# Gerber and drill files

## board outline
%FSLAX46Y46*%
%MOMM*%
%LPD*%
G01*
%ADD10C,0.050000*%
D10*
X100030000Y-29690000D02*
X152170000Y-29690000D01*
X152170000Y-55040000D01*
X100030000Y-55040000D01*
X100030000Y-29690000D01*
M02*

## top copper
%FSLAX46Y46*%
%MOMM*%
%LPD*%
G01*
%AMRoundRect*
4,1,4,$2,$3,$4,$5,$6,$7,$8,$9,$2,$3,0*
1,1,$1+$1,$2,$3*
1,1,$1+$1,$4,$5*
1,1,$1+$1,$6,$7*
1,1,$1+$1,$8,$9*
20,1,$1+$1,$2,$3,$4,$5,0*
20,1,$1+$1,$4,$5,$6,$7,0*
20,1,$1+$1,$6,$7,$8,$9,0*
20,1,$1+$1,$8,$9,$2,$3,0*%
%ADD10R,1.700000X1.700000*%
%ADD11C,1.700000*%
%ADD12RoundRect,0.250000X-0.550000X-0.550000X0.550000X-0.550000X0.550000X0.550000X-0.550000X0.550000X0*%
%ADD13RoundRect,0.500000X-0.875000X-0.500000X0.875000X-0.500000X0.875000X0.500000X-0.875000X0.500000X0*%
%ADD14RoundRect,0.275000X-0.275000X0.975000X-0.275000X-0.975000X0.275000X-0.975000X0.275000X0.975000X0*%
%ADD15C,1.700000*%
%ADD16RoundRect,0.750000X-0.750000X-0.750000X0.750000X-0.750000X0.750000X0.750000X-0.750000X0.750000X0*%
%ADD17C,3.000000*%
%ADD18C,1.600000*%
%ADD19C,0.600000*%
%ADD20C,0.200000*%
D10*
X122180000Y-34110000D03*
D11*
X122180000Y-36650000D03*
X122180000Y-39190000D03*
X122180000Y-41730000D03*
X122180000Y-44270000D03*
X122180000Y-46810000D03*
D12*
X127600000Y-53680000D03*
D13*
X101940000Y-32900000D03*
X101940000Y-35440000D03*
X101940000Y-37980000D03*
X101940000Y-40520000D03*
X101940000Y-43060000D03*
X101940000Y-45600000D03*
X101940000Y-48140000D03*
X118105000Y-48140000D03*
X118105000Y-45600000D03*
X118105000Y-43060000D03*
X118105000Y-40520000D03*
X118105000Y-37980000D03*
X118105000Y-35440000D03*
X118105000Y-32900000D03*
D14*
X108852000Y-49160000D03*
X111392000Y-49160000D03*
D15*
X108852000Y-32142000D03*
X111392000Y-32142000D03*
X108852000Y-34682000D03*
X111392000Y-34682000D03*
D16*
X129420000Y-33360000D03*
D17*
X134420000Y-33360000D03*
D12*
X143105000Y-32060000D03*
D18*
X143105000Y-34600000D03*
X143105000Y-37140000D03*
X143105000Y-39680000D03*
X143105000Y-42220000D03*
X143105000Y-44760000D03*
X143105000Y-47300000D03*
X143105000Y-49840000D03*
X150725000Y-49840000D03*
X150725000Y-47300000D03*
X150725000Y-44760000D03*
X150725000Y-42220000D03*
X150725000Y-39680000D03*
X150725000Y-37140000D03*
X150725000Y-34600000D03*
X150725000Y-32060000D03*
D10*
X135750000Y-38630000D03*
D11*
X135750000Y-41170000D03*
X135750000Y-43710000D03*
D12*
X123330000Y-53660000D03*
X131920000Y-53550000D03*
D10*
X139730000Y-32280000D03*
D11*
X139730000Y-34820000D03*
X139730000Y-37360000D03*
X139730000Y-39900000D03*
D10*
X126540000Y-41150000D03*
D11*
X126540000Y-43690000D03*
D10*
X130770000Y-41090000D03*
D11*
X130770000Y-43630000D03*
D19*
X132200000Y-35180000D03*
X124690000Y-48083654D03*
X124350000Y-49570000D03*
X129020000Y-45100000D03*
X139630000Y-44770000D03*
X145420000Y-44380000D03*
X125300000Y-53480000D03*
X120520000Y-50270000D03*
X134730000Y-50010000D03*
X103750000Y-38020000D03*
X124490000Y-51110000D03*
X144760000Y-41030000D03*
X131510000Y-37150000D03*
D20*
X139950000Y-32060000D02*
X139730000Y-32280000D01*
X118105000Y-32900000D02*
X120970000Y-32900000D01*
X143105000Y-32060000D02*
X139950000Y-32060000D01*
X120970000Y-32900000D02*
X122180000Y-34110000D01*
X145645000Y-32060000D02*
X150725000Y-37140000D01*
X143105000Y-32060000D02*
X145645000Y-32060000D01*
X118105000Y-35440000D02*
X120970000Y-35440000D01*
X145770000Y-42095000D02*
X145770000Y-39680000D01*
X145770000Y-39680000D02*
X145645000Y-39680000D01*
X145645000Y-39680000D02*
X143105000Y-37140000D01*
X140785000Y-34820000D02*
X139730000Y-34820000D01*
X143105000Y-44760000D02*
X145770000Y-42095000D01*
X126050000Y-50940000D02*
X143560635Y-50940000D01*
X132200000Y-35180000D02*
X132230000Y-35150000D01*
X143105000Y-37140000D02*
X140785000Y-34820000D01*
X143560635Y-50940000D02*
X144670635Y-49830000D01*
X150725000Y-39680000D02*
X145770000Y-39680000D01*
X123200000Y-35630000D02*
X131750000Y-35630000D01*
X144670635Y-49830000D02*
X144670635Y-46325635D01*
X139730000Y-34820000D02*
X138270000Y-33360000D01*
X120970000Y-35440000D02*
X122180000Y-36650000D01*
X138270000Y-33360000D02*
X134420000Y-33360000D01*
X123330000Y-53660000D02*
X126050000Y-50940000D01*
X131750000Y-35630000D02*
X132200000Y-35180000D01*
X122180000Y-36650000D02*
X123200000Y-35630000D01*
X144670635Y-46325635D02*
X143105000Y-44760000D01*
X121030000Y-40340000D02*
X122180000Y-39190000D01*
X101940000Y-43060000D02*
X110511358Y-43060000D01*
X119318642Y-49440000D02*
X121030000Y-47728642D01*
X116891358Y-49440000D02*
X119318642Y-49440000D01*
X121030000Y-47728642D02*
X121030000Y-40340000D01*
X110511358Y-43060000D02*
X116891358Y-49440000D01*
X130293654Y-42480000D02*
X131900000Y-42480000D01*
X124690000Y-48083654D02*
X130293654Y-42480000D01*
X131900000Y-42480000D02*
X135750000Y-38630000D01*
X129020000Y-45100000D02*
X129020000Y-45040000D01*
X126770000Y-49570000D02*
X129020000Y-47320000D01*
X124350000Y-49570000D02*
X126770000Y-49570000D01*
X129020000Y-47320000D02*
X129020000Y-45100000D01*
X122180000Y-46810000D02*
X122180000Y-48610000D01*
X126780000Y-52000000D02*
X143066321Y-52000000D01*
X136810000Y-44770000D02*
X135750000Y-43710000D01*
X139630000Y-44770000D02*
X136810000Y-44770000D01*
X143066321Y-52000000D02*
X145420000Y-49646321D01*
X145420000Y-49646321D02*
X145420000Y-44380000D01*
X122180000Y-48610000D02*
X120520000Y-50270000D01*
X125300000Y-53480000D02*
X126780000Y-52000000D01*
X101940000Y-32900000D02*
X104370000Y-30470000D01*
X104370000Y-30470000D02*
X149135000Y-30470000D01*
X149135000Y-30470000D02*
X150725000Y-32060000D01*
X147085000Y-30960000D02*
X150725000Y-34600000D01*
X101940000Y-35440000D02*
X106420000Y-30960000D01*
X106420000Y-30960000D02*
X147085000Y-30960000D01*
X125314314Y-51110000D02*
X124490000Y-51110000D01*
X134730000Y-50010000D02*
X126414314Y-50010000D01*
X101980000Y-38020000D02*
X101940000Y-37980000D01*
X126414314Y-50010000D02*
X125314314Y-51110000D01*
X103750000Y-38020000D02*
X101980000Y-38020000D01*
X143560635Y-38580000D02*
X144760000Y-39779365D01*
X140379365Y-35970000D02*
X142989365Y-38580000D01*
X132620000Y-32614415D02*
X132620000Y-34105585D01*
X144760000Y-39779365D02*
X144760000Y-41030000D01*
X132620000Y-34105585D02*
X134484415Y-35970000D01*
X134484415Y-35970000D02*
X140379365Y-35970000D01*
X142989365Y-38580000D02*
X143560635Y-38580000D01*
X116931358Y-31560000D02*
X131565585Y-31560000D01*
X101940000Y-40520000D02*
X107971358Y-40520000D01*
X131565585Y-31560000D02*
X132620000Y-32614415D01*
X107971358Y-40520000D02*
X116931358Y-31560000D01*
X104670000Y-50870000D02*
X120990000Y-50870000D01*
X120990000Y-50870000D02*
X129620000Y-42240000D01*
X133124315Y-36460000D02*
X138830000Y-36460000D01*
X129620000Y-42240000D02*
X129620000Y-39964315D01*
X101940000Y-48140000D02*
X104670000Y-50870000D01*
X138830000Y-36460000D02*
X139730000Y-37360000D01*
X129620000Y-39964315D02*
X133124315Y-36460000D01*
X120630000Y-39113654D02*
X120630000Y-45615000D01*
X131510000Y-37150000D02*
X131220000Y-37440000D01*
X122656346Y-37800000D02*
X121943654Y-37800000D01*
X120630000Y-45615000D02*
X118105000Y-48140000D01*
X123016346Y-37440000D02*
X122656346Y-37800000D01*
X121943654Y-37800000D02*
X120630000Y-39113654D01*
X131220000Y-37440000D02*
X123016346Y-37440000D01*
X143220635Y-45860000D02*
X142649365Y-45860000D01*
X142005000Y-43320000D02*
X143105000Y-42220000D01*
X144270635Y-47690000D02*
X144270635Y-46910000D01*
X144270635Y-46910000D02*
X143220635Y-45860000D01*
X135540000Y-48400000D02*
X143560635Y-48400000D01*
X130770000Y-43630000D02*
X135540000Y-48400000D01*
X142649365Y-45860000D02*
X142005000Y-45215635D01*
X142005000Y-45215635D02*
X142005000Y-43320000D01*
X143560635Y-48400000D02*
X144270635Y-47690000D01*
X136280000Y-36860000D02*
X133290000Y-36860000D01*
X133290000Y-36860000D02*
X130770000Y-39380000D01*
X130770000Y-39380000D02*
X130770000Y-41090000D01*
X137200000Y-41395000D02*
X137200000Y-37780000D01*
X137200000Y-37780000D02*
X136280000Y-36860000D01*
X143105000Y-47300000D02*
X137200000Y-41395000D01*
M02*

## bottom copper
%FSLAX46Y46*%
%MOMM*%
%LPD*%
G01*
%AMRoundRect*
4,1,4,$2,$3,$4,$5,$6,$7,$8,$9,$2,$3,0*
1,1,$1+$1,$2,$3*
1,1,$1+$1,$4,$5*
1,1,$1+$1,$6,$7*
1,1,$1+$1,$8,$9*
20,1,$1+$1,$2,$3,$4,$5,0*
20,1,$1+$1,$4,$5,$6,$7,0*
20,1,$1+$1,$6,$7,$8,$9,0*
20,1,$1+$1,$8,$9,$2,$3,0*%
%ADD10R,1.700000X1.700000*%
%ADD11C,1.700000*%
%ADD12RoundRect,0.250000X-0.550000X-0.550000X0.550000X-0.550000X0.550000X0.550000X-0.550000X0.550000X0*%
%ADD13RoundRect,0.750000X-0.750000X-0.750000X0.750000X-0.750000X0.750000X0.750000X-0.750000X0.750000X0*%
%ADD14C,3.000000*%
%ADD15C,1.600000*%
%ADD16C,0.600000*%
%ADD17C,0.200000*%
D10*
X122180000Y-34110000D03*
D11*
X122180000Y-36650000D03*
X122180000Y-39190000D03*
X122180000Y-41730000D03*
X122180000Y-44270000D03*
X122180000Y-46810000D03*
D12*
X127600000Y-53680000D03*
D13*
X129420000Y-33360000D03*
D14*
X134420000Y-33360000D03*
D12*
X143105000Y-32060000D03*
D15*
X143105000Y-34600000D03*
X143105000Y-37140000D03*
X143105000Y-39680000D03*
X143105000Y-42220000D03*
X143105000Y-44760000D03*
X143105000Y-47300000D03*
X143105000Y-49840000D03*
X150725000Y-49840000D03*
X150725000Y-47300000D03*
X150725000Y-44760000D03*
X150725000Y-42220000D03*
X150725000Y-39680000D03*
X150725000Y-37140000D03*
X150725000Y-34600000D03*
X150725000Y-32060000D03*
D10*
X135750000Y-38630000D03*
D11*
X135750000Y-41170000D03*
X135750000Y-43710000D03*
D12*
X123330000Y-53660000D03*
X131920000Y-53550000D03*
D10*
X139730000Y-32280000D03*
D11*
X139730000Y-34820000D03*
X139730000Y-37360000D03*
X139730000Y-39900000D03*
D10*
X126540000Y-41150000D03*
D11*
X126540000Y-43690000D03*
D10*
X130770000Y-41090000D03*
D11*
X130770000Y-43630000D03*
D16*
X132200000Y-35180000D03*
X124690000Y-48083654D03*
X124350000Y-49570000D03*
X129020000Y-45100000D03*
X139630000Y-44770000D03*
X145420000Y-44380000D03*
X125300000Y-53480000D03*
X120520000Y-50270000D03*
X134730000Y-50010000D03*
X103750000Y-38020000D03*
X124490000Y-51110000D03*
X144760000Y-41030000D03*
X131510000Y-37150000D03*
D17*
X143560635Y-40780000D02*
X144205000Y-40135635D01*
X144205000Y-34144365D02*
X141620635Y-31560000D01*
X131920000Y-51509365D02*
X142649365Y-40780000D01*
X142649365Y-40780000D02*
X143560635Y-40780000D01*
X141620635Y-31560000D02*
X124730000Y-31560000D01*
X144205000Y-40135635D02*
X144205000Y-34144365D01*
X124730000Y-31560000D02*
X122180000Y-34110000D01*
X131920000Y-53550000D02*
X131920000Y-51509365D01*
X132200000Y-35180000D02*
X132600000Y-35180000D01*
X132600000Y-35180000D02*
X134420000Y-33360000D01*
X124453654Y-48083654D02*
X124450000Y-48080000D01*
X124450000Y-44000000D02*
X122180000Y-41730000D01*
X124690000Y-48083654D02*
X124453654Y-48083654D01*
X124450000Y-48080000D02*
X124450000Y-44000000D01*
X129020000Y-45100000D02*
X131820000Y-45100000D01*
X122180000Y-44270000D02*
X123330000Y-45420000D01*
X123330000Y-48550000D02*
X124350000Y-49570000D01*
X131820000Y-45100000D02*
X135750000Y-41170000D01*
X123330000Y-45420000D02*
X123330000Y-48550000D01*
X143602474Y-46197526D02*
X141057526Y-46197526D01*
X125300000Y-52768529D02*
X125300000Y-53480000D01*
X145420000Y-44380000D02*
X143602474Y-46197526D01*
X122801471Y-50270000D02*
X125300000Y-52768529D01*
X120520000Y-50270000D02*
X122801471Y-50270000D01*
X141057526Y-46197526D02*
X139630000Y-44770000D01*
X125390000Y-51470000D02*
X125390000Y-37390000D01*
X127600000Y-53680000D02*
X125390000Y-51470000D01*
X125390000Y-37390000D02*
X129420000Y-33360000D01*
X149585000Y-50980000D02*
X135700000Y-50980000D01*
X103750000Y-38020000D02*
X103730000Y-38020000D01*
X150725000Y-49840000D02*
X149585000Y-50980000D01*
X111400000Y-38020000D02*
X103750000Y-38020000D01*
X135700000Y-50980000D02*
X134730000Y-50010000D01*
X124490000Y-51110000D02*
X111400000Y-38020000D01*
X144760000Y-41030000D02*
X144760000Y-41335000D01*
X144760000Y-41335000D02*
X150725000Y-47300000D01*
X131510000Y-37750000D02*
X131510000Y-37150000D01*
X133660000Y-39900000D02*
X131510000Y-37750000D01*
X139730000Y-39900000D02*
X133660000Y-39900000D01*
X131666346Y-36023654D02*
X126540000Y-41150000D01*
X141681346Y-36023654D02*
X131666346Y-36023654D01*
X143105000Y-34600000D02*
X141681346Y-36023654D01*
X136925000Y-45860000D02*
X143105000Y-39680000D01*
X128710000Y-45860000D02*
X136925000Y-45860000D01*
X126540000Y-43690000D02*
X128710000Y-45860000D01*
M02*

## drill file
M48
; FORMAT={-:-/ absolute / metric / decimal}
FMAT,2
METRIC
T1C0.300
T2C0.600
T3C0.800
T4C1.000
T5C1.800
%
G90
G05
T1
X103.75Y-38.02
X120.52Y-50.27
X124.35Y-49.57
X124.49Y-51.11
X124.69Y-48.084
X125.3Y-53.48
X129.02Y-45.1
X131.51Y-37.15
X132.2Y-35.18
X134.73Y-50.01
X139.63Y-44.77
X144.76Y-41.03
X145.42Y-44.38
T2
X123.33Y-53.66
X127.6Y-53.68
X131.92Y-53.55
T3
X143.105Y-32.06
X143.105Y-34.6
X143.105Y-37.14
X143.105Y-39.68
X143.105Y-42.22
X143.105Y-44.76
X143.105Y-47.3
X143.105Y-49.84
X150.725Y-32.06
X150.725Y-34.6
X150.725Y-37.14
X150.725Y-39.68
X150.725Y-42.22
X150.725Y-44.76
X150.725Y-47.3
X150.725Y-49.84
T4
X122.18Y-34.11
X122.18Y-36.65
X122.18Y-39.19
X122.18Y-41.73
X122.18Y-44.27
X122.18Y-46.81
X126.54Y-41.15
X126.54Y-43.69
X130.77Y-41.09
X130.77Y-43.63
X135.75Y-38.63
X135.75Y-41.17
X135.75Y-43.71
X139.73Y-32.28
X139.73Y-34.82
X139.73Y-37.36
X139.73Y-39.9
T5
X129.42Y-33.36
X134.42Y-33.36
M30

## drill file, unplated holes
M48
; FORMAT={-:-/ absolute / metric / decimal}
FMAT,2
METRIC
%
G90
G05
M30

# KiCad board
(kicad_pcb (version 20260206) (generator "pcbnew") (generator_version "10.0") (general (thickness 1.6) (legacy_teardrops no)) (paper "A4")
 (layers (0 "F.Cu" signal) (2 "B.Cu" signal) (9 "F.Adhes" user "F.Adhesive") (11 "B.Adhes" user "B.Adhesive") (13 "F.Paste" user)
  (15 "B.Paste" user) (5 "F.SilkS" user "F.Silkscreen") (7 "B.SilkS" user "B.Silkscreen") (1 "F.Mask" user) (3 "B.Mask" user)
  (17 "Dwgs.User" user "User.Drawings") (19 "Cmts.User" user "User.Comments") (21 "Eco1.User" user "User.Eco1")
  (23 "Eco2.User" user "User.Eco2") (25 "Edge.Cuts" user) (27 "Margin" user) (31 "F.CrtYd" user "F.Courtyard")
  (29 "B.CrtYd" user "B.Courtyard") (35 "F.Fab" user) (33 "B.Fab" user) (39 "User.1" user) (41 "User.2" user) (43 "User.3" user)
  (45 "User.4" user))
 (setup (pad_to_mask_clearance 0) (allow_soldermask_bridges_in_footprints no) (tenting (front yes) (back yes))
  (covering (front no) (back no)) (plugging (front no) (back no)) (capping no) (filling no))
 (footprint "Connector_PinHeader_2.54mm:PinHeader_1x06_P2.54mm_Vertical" (layer "F.Cu") (at 122.18 34.11)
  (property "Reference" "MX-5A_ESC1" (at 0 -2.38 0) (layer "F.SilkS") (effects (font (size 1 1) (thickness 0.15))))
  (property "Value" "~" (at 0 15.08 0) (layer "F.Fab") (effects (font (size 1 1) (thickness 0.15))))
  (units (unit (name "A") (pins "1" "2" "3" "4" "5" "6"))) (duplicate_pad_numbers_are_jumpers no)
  (pad "1" thru_hole rect (at 0 0) (size 1.7 1.7) (drill 1) (layers "*.Cu" "*.Mask") (remove_unused_layers no) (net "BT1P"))
  (pad "2" thru_hole circle (at 0 2.54) (size 1.7 1.7) (drill 1) (layers "*.Cu" "*.Mask") (remove_unused_layers no) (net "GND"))
  (pad "3" thru_hole circle (at 0 5.08) (size 1.7 1.7) (drill 1) (layers "*.Cu" "*.Mask") (remove_unused_layers no)
   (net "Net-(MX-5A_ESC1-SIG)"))
  (pad "4" thru_hole circle (at 0 7.62) (size 1.7 1.7) (drill 1) (layers "*.Cu" "*.Mask") (remove_unused_layers no)
   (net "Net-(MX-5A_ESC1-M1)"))
  (pad "5" thru_hole circle (at 0 10.16) (size 1.7 1.7) (drill 1) (layers "*.Cu" "*.Mask") (remove_unused_layers no)
   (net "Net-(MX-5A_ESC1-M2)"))
  (pad "6" thru_hole circle (at 0 12.7) (size 1.7 1.7) (drill 1) (layers "*.Cu" "*.Mask") (remove_unused_layers no)
   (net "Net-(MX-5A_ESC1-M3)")))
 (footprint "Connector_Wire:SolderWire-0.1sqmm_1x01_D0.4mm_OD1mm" (layer "F.Cu") (at 127.6 53.68)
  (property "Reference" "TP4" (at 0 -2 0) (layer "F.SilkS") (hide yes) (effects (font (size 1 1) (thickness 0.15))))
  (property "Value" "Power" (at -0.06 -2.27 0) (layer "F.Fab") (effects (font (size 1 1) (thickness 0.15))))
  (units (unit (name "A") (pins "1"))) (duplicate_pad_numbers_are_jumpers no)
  (pad "1" thru_hole roundrect (at 0 0) (size 1.6 1.6) (drill 0.6) (layers "*.Cu" "*.Mask") (remove_unused_layers no)
   (roundrect_rratio 0.15625) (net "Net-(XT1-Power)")))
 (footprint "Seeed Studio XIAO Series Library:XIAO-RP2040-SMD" (layer "F.Cu") (at 109.94 40.52)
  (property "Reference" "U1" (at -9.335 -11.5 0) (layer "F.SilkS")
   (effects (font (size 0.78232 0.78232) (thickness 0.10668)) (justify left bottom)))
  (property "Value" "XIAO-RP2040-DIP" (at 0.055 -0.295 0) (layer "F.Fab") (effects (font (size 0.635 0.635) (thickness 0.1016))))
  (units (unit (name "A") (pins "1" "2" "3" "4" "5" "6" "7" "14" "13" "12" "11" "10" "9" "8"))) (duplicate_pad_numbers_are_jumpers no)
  (pad "1" smd roundrect (at -8 -7.62) (size 2.75 2) (layers "F.Cu" "F.Mask" "F.Paste") (roundrect_rratio 0.25) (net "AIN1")
   (solder_mask_margin 0.0508) (thermal_bridge_angle 45))
  (pad "2" smd roundrect (at -8 -5.08) (size 2.75 2) (layers "F.Cu" "F.Mask" "F.Paste") (roundrect_rratio 0.25) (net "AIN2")
   (solder_mask_margin 0.0508) (thermal_bridge_angle 45))
  (pad "3" smd roundrect (at -8 -2.54) (size 2.75 2) (layers "F.Cu" "F.Mask" "F.Paste") (roundrect_rratio 0.25) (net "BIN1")
   (solder_mask_margin 0.0508) (thermal_bridge_angle 45))
  (pad "4" smd roundrect (at -8 0) (size 2.75 2) (layers "F.Cu" "F.Mask" "F.Paste") (roundrect_rratio 0.25) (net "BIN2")
   (solder_mask_margin 0.0508) (thermal_bridge_angle 45))
  (pad "5" smd roundrect (at -8 2.54) (size 2.75 2) (layers "F.Cu" "F.Mask" "F.Paste") (roundrect_rratio 0.25) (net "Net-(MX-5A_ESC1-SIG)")
   (solder_mask_margin 0.0508) (thermal_bridge_angle 45))
  (pad "6" smd roundrect (at -8 5.08) (size 2.75 2) (layers "F.Cu" "F.Mask" "F.Paste") (roundrect_rratio 0.25)
   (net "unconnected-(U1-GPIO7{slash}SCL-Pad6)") (solder_mask_margin 0.0508) (thermal_bridge_angle 45))
  (pad "7" smd roundrect (at -8 7.62) (size 2.75 2) (layers "F.Cu" "F.Mask" "F.Paste") (roundrect_rratio 0.25)
   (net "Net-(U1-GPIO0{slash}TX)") (solder_mask_margin 0.0508) (thermal_bridge_angle 45))
  (pad "8" smd roundrect (at 8.165 7.62) (size 2.75 2) (layers "F.Cu" "F.Mask" "F.Paste") (roundrect_rratio 0.25)
   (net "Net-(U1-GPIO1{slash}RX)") (solder_mask_margin 0.0508) (thermal_bridge_angle 45))
  (pad "9" smd roundrect (at 8.165 5.08) (size 2.75 2) (layers "F.Cu" "F.Mask" "F.Paste") (roundrect_rratio 0.25)
   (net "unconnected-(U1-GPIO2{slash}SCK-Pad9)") (solder_mask_margin 0.0508) (thermal_bridge_angle 45))
  (pad "10" smd roundrect (at 8.165 2.54) (size 2.75 2) (layers "F.Cu" "F.Mask" "F.Paste") (roundrect_rratio 0.25)
   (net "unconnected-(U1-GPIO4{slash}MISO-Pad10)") (solder_mask_margin 0.0508) (thermal_bridge_angle 45))
  (pad "11" smd roundrect (at 8.165 0) (size 2.75 2) (layers "F.Cu" "F.Mask" "F.Paste") (roundrect_rratio 0.25)
   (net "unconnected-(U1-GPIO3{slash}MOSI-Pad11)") (solder_mask_margin 0.0508) (thermal_bridge_angle 45))
  (pad "12" smd roundrect (at 8.165 -2.54) (size 2.75 2) (layers "F.Cu" "F.Mask" "F.Paste") (roundrect_rratio 0.25)
   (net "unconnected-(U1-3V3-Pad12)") (solder_mask_margin 0.0508) (thermal_bridge_angle 45))
  (pad "13" smd roundrect (at 8.165 -5.08) (size 2.75 2) (layers "F.Cu" "F.Mask" "F.Paste") (roundrect_rratio 0.25) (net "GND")
   (solder_mask_margin 0.0508) (thermal_bridge_angle 45))
  (pad "14" smd roundrect (at 8.165 -7.62) (size 2.75 2) (layers "F.Cu" "F.Mask" "F.Paste") (roundrect_rratio 0.25) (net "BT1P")
   (solder_mask_margin 0.0508) (thermal_bridge_angle 45))
  (pad "15" smd roundrect (at -1.088 8.64 270) (size 2.5 1.1) (layers "F.Cu" "F.Mask" "F.Paste") (roundrect_rratio 0.25)
   (thermal_bridge_angle 45))
  (pad "16" smd roundrect (at 1.452 8.64 270) (size 2.5 1.1) (layers "F.Cu" "F.Mask" "F.Paste") (roundrect_rratio 0.25)
   (thermal_bridge_angle 45))
  (pad "17" smd circle (at -1.088 -8.378) (size 1.7 1.7) (layers "F.Cu" "F.Mask" "F.Paste"))
  (pad "18" smd circle (at 1.452 -8.378) (size 1.7 1.7) (layers "F.Cu" "F.Mask" "F.Paste"))
  (pad "19" smd circle (at -1.088 -5.838) (size 1.7 1.7) (layers "F.Cu" "F.Mask" "F.Paste"))
  (pad "20" smd circle (at 1.452 -5.838) (size 1.7 1.7) (layers "F.Cu" "F.Mask" "F.Paste")))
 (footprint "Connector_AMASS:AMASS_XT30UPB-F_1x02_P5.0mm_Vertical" (layer "F.Cu") (at 129.42 33.36)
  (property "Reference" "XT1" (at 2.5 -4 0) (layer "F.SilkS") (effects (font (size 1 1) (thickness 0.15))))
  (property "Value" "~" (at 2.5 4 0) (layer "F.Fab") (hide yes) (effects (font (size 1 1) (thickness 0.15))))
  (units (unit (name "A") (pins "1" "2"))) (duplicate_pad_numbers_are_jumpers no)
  (pad "1" thru_hole roundrect (at 0 0) (size 3 3) (drill 1.8) (layers "*.Cu" "*.Mask") (remove_unused_layers no) (roundrect_rratio 0.25)
   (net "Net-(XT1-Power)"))
  (pad "2" thru_hole circle (at 5 0) (size 3 3) (drill 1.8) (layers "*.Cu" "*.Mask") (remove_unused_layers no) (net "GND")))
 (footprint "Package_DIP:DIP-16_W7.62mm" (layer "F.Cu") (at 143.105 32.06)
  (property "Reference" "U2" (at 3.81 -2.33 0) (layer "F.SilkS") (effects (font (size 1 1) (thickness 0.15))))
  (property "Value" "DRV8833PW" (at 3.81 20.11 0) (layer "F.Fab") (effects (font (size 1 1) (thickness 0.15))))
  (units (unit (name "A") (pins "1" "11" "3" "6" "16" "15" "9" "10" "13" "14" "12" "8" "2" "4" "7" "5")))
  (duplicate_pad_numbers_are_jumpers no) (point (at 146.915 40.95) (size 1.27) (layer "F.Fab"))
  (pad "1" thru_hole roundrect (at 0 0) (size 1.6 1.6) (drill 0.8) (layers "*.Cu" "*.Mask") (remove_unused_layers no)
   (roundrect_rratio 0.15625) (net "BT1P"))
  (pad "2" thru_hole circle (at 0 2.54) (size 1.6 1.6) (drill 0.8) (layers "*.Cu" "*.Mask") (remove_unused_layers no) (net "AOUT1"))
  (pad "3" thru_hole circle (at 0 5.08) (size 1.6 1.6) (drill 0.8) (layers "*.Cu" "*.Mask") (remove_unused_layers no) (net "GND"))
  (pad "4" thru_hole circle (at 0 7.62) (size 1.6 1.6) (drill 0.8) (layers "*.Cu" "*.Mask") (remove_unused_layers no) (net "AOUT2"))
  (pad "5" thru_hole circle (at 0 10.16) (size 1.6 1.6) (drill 0.8) (layers "*.Cu" "*.Mask") (remove_unused_layers no) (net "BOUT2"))
  (pad "6" thru_hole circle (at 0 12.7) (size 1.6 1.6) (drill 0.8) (layers "*.Cu" "*.Mask") (remove_unused_layers no) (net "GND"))
  (pad "7" thru_hole circle (at 0 15.24) (size 1.6 1.6) (drill 0.8) (layers "*.Cu" "*.Mask") (remove_unused_layers no) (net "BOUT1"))
  (pad "8" thru_hole circle (at 0 17.78) (size 1.6 1.6) (drill 0.8) (layers "*.Cu" "*.Mask") (remove_unused_layers no)
   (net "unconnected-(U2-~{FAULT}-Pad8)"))
  (pad "9" thru_hole circle (at 7.62 17.78) (size 1.6 1.6) (drill 0.8) (layers "*.Cu" "*.Mask") (remove_unused_layers no) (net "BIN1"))
  (pad "10" thru_hole circle (at 7.62 15.24) (size 1.6 1.6) (drill 0.8) (layers "*.Cu" "*.Mask") (remove_unused_layers no) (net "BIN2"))
  (pad "11" thru_hole circle (at 7.62 12.7) (size 1.6 1.6) (drill 0.8) (layers "*.Cu" "*.Mask") (remove_unused_layers no)
   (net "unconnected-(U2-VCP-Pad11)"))
  (pad "12" thru_hole circle (at 7.62 10.16) (size 1.6 1.6) (drill 0.8) (layers "*.Cu" "*.Mask") (remove_unused_layers no)
   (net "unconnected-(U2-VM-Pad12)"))
  (pad "13" thru_hole circle (at 7.62 7.62) (size 1.6 1.6) (drill 0.8) (layers "*.Cu" "*.Mask") (remove_unused_layers no) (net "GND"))
  (pad "14" thru_hole circle (at 7.62 5.08) (size 1.6 1.6) (drill 0.8) (layers "*.Cu" "*.Mask") (remove_unused_layers no) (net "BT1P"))
  (pad "15" thru_hole circle (at 7.62 2.54) (size 1.6 1.6) (drill 0.8) (layers "*.Cu" "*.Mask") (remove_unused_layers no) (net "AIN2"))
  (pad "16" thru_hole circle (at 7.62 0) (size 1.6 1.6) (drill 0.8) (layers "*.Cu" "*.Mask") (remove_unused_layers no) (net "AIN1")))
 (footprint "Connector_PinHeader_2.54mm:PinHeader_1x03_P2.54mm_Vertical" (layer "F.Cu") (at 135.75 38.63)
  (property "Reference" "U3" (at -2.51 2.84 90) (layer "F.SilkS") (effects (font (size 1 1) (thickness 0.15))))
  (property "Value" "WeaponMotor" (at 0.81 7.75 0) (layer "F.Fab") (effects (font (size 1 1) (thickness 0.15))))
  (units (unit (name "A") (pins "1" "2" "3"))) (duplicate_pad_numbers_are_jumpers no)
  (pad "1" thru_hole rect (at 0 0) (size 1.7 1.7) (drill 1) (layers "*.Cu" "*.Mask") (remove_unused_layers no) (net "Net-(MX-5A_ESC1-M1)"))
  (pad "2" thru_hole circle (at 0 2.54) (size 1.7 1.7) (drill 1) (layers "*.Cu" "*.Mask") (remove_unused_layers no)
   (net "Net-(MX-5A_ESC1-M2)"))
  (pad "3" thru_hole circle (at 0 5.08) (size 1.7 1.7) (drill 1) (layers "*.Cu" "*.Mask") (remove_unused_layers no)
   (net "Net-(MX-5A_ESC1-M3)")))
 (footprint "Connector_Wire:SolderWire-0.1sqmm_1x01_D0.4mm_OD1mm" (layer "F.Cu") (at 123.33 53.66)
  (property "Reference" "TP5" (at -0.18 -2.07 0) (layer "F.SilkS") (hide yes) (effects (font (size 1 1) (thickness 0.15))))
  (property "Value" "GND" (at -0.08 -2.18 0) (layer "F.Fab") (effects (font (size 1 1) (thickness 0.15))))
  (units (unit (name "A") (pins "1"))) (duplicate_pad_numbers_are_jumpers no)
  (pad "1" thru_hole roundrect (at 0 0) (size 1.6 1.6) (drill 0.6) (layers "*.Cu" "*.Mask") (remove_unused_layers no)
   (roundrect_rratio 0.15625) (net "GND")))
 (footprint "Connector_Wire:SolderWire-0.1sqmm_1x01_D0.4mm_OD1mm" (layer "F.Cu") (at 131.92 53.55)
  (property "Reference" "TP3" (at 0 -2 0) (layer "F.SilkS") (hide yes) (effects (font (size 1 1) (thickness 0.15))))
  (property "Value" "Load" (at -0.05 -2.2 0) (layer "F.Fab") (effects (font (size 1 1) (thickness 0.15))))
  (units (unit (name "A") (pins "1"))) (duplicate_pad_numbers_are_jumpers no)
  (pad "1" thru_hole roundrect (at 0 0) (size 1.6 1.6) (drill 0.6) (layers "*.Cu" "*.Mask") (remove_unused_layers no)
   (roundrect_rratio 0.15625) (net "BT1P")))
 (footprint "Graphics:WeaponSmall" (layer "F.Cu") (at 103.49791 55.032445 90)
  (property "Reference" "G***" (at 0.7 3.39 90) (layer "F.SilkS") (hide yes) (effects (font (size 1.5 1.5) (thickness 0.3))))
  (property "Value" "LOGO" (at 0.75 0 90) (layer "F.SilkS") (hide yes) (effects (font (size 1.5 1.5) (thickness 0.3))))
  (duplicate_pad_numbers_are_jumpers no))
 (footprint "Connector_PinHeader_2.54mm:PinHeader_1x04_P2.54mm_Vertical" (layer "F.Cu") (at 139.73 32.28)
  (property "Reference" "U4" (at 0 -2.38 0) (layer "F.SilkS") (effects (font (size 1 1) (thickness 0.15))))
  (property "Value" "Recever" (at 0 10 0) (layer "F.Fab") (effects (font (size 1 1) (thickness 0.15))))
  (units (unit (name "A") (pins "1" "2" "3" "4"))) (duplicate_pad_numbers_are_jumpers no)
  (pad "1" thru_hole rect (at 0 0) (size 1.7 1.7) (drill 1) (layers "*.Cu" "*.Mask") (remove_unused_layers no) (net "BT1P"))
  (pad "2" thru_hole circle (at 0 2.54) (size 1.7 1.7) (drill 1) (layers "*.Cu" "*.Mask") (remove_unused_layers no) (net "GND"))
  (pad "3" thru_hole circle (at 0 5.08) (size 1.7 1.7) (drill 1) (layers "*.Cu" "*.Mask") (remove_unused_layers no)
   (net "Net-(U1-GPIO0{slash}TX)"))
  (pad "4" thru_hole circle (at 0 7.62) (size 1.7 1.7) (drill 1) (layers "*.Cu" "*.Mask") (remove_unused_layers no)
   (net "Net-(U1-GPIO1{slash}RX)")))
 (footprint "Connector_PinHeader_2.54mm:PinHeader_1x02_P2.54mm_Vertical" (layer "F.Cu") (at 126.54 41.15)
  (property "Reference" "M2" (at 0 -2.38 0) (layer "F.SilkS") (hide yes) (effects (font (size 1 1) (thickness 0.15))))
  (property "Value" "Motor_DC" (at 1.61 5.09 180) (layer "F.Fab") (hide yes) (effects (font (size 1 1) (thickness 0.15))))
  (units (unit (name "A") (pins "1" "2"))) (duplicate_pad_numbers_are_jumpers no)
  (pad "1" thru_hole rect (at 0 0) (size 1.7 1.7) (drill 1) (layers "*.Cu" "*.Mask") (remove_unused_layers no) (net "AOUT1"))
  (pad "2" thru_hole circle (at 0 2.54) (size 1.7 1.7) (drill 1) (layers "*.Cu" "*.Mask") (remove_unused_layers no) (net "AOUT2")))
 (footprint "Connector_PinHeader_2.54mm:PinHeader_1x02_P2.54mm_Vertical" (layer "F.Cu") (at 130.77 41.09)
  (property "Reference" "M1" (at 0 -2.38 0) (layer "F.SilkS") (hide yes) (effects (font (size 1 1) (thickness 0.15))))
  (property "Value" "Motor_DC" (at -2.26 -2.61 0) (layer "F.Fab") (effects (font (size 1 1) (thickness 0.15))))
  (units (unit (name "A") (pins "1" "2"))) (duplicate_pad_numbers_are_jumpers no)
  (pad "1" thru_hole rect (at 0 0) (size 1.7 1.7) (drill 1) (layers "*.Cu" "*.Mask") (remove_unused_layers no) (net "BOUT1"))
  (pad "2" thru_hole circle (at 0 2.54) (size 1.7 1.7) (drill 1) (layers "*.Cu" "*.Mask") (remove_unused_layers no) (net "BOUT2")))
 (gr_rect (start 100.03 29.69) (end 152.17 55.04) (stroke (width 0.05) (type default)) (fill no) (layer "Edge.Cuts"))
 (segment (start 139.95 32.06) (end 139.73 32.28) (width 0.2) (layer "F.Cu") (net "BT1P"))
 (segment (start 118.105 32.9) (end 120.97 32.9) (width 0.2) (layer "F.Cu") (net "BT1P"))
 (segment (start 143.105 32.06) (end 139.95 32.06) (width 0.2) (layer "F.Cu") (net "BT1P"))
 (segment (start 120.97 32.9) (end 122.18 34.11) (width 0.2) (layer "F.Cu") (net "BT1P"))
 (segment (start 145.645 32.06) (end 150.725 37.14) (width 0.2) (layer "F.Cu") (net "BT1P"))
 (segment (start 143.105 32.06) (end 145.645 32.06) (width 0.2) (layer "F.Cu") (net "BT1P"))
 (segment (start 143.560635 40.78) (end 144.205 40.135635) (width 0.2) (layer "B.Cu") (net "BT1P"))
 (segment (start 144.205 34.144365) (end 141.620635 31.56) (width 0.2) (layer "B.Cu") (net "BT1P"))
 (segment (start 131.92 51.509365) (end 142.649365 40.78) (width 0.2) (layer "B.Cu") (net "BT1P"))
 (segment (start 142.649365 40.78) (end 143.560635 40.78) (width 0.2) (layer "B.Cu") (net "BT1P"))
 (segment (start 141.620635 31.56) (end 124.73 31.56) (width 0.2) (layer "B.Cu") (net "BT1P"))
 (segment (start 144.205 40.135635) (end 144.205 34.144365) (width 0.2) (layer "B.Cu") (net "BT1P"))
 (segment (start 124.73 31.56) (end 122.18 34.11) (width 0.2) (layer "B.Cu") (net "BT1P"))
 (segment (start 131.92 53.55) (end 131.92 51.509365) (width 0.2) (layer "B.Cu") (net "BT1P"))
 (segment (start 118.105 35.44) (end 120.97 35.44) (width 0.2) (layer "F.Cu") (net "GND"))
 (segment (start 145.77 42.095) (end 145.77 39.68) (width 0.2) (layer "F.Cu") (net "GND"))
 (segment (start 145.77 39.68) (end 145.645 39.68) (width 0.2) (layer "F.Cu") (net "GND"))
 (segment (start 145.645 39.68) (end 143.105 37.14) (width 0.2) (layer "F.Cu") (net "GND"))
 (segment (start 140.785 34.82) (end 139.73 34.82) (width 0.2) (layer "F.Cu") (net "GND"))
 (segment (start 143.105 44.76) (end 145.77 42.095) (width 0.2) (layer "F.Cu") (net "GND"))
 (segment (start 126.05 50.94) (end 143.560635 50.94) (width 0.2) (layer "F.Cu") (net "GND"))
 (segment (start 132.2 35.18) (end 132.23 35.15) (width 0.2) (layer "F.Cu") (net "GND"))
 (segment (start 143.105 37.14) (end 140.785 34.82) (width 0.2) (layer "F.Cu") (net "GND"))
 (segment (start 143.560635 50.94) (end 144.670635 49.83) (width 0.2) (layer "F.Cu") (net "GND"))
 (segment (start 150.725 39.68) (end 145.77 39.68) (width 0.2) (layer "F.Cu") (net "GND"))
 (segment (start 123.2 35.63) (end 131.75 35.63) (width 0.2) (layer "F.Cu") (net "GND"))
 (segment (start 144.670635 49.83) (end 144.670635 46.325635) (width 0.2) (layer "F.Cu") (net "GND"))
 (segment (start 139.73 34.82) (end 138.27 33.36) (width 0.2) (layer "F.Cu") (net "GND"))
 (segment (start 120.97 35.44) (end 122.18 36.65) (width 0.2) (layer "F.Cu") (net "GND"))
 (segment (start 138.27 33.36) (end 134.42 33.36) (width 0.2) (layer "F.Cu") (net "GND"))
 (segment (start 123.33 53.66) (end 126.05 50.94) (width 0.2) (layer "F.Cu") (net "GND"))
 (segment (start 131.75 35.63) (end 132.2 35.18) (width 0.2) (layer "F.Cu") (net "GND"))
 (segment (start 122.18 36.65) (end 123.2 35.63) (width 0.2) (layer "F.Cu") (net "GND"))
 (segment (start 144.670635 46.325635) (end 143.105 44.76) (width 0.2) (layer "F.Cu") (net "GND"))
 (via (at 132.2 35.18) (size 0.6) (drill 0.3) (layers "F.Cu" "B.Cu") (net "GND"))
 (segment (start 132.2 35.18) (end 132.6 35.18) (width 0.2) (layer "B.Cu") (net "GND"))
 (segment (start 132.6 35.18) (end 134.42 33.36) (width 0.2) (layer "B.Cu") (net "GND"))
 (segment (start 121.03 40.34) (end 122.18 39.19) (width 0.2) (layer "F.Cu") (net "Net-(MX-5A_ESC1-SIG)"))
 (segment (start 101.94 43.06) (end 110.511358 43.06) (width 0.2) (layer "F.Cu") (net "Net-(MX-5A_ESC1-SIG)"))
 (segment (start 119.318642 49.44) (end 121.03 47.728642) (width 0.2) (layer "F.Cu") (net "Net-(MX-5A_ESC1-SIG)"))
 (segment (start 116.891358 49.44) (end 119.318642 49.44) (width 0.2) (layer "F.Cu") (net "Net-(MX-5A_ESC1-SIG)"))
 (segment (start 121.03 47.728642) (end 121.03 40.34) (width 0.2) (layer "F.Cu") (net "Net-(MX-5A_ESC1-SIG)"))
 (segment (start 110.511358 43.06) (end 116.891358 49.44) (width 0.2) (layer "F.Cu") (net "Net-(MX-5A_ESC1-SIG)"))
 (segment (start 130.293654 42.48) (end 131.9 42.48) (width 0.2) (layer "F.Cu") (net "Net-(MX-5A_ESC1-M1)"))
 (segment (start 124.69 48.083654) (end 130.293654 42.48) (width 0.2) (layer "F.Cu") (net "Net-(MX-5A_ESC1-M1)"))
 (segment (start 131.9 42.48) (end 135.75 38.63) (width 0.2) (layer "F.Cu") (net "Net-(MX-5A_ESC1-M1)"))
 (via (at 124.69 48.083654) (size 0.6) (drill 0.3) (layers "F.Cu" "B.Cu") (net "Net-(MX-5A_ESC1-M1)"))
 (segment (start 124.453654 48.083654) (end 124.45 48.08) (width 0.2) (layer "B.Cu") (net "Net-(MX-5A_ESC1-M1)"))
 (segment (start 124.45 44) (end 122.18 41.73) (width 0.2) (layer "B.Cu") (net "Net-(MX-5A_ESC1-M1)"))
 (segment (start 124.69 48.083654) (end 124.453654 48.083654) (width 0.2) (layer "B.Cu") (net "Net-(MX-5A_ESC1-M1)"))
 (segment (start 124.45 48.08) (end 124.45 44) (width 0.2) (layer "B.Cu") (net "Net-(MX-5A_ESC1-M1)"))
 (segment (start 129.02 45.1) (end 129.02 45.04) (width 0.2) (layer "F.Cu") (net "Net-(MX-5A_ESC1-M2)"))
 (segment (start 126.77 49.57) (end 129.02 47.32) (width 0.2) (layer "F.Cu") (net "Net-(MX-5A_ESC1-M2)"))
 (segment (start 124.35 49.57) (end 126.77 49.57) (width 0.2) (layer "F.Cu") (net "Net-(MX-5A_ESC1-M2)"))
 (segment (start 129.02 47.32) (end 129.02 45.1) (width 0.2) (layer "F.Cu") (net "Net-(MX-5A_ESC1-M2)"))
 (via (at 124.35 49.57) (size 0.6) (drill 0.3) (layers "F.Cu" "B.Cu") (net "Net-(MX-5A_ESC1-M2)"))
 (via (at 129.02 45.1) (size 0.6) (drill 0.3) (layers "F.Cu" "B.Cu") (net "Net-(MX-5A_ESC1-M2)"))
 (segment (start 129.02 45.1) (end 131.82 45.1) (width 0.2) (layer "B.Cu") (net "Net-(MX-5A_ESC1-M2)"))
 (segment (start 122.18 44.27) (end 123.33 45.42) (width 0.2) (layer "B.Cu") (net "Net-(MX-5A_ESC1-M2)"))
 (segment (start 123.33 48.55) (end 124.35 49.57) (width 0.2) (layer "B.Cu") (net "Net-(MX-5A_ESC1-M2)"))
 (segment (start 131.82 45.1) (end 135.75 41.17) (width 0.2) (layer "B.Cu") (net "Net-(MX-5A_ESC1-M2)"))
 (segment (start 123.33 45.42) (end 123.33 48.55) (width 0.2) (layer "B.Cu") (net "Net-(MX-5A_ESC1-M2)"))
 (segment (start 122.18 46.81) (end 122.18 48.61) (width 0.2) (layer "F.Cu") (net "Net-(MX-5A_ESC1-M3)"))
 (segment (start 126.78 52) (end 143.066321 52) (width 0.2) (layer "F.Cu") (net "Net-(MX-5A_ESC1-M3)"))
 (segment (start 136.81 44.77) (end 135.75 43.71) (width 0.2) (layer "F.Cu") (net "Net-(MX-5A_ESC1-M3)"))
 (segment (start 139.63 44.77) (end 136.81 44.77) (width 0.2) (layer "F.Cu") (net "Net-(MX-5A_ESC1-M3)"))
 (segment (start 143.066321 52) (end 145.42 49.646321) (width 0.2) (layer "F.Cu") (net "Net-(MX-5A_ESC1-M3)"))
 (segment (start 145.42 49.646321) (end 145.42 44.38) (width 0.2) (layer "F.Cu") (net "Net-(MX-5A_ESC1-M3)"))
 (segment (start 122.18 48.61) (end 120.52 50.27) (width 0.2) (layer "F.Cu") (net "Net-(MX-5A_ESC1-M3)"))
 (segment (start 125.3 53.48) (end 126.78 52) (width 0.2) (layer "F.Cu") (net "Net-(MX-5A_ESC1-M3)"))
 (via (at 139.63 44.77) (size 0.6) (drill 0.3) (layers "F.Cu" "B.Cu") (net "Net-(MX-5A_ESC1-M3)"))
 (via (at 145.42 44.38) (size 0.6) (drill 0.3) (layers "F.Cu" "B.Cu") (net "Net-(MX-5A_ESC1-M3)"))
 (via (at 125.3 53.48) (size 0.6) (drill 0.3) (layers "F.Cu" "B.Cu") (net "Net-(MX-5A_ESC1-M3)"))
 (via (at 120.52 50.27) (size 0.6) (drill 0.3) (layers "F.Cu" "B.Cu") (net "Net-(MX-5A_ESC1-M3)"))
 (segment (start 143.602474 46.197526) (end 141.057526 46.197526) (width 0.2) (layer "B.Cu") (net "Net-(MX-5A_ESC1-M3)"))
 (segment (start 125.3 52.768529) (end 125.3 53.48) (width 0.2) (layer "B.Cu") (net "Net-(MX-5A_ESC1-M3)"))
 (segment (start 145.42 44.38) (end 143.602474 46.197526) (width 0.2) (layer "B.Cu") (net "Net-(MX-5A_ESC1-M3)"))
 (segment (start 122.801471 50.27) (end 125.3 52.768529) (width 0.2) (layer "B.Cu") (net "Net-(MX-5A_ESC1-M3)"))
 (segment (start 120.52 50.27) (end 122.801471 50.27) (width 0.2) (layer "B.Cu") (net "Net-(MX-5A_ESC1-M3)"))
 (segment (start 141.057526 46.197526) (end 139.63 44.77) (width 0.2) (layer "B.Cu") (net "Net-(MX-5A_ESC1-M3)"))
 (segment (start 125.39 51.47) (end 125.39 37.39) (width 0.2) (layer "B.Cu") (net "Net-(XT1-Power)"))
 (segment (start 127.6 53.68) (end 125.39 51.47) (width 0.2) (layer "B.Cu") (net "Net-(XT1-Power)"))
 (segment (start 125.39 37.39) (end 129.42 33.36) (width 0.2) (layer "B.Cu") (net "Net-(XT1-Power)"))
 (segment (start 101.94 32.9) (end 104.37 30.47) (width 0.2) (layer "F.Cu") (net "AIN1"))
 (segment (start 104.37 30.47) (end 149.135 30.47) (width 0.2) (layer "F.Cu") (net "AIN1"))
 (segment (start 149.135 30.47) (end 150.725 32.06) (width 0.2) (layer "F.Cu") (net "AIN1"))
 (segment (start 147.085 30.96) (end 150.725 34.6) (width 0.2) (layer "F.Cu") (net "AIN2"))
 (segment (start 101.94 35.44) (end 106.42 30.96) (width 0.2) (layer "F.Cu") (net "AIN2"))
 (segment (start 106.42 30.96) (end 147.085 30.96) (width 0.2) (layer "F.Cu") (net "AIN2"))
 (segment (start 125.314314 51.11) (end 124.49 51.11) (width 0.2) (layer "F.Cu") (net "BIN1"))
 (segment (start 134.73 50.01) (end 126.414314 50.01) (width 0.2) (layer "F.Cu") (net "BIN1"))
 (segment (start 101.98 38.02) (end 101.94 37.98) (width 0.2) (layer "F.Cu") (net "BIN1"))
 (segment (start 126.414314 50.01) (end 125.314314 51.11) (width 0.2) (layer "F.Cu") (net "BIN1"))
 (segment (start 103.75 38.02) (end 101.98 38.02) (width 0.2) (layer "F.Cu") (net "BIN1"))
 (via (at 134.73 50.01) (size 0.6) (drill 0.3) (layers "F.Cu" "B.Cu") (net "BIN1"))
 (via (at 103.75 38.02) (size 0.6) (drill 0.3) (layers "F.Cu" "B.Cu") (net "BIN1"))
 (via (at 124.49 51.11) (size 0.6) (drill 0.3) (layers "F.Cu" "B.Cu") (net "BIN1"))
 (segment (start 149.585 50.98) (end 135.7 50.98) (width 0.2) (layer "B.Cu") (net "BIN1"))
 (segment (start 103.75 38.02) (end 103.73 38.02) (width 0.2) (layer "B.Cu") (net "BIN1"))
 (segment (start 150.725 49.84) (end 149.585 50.98) (width 0.2) (layer "B.Cu") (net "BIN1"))
 (segment (start 111.4 38.02) (end 103.75 38.02) (width 0.2) (layer "B.Cu") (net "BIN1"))
 (segment (start 135.7 50.98) (end 134.73 50.01) (width 0.2) (layer "B.Cu") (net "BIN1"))
 (segment (start 124.49 51.11) (end 111.4 38.02) (width 0.2) (layer "B.Cu") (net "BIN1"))
 (segment (start 143.560635 38.58) (end 144.76 39.779365) (width 0.2) (layer "F.Cu") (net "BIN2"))
 (segment (start 140.379365 35.97) (end 142.989365 38.58) (width 0.2) (layer "F.Cu") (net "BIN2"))
 (segment (start 132.62 32.614415) (end 132.62 34.105585) (width 0.2) (layer "F.Cu") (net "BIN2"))
 (segment (start 144.76 39.779365) (end 144.76 41.03) (width 0.2) (layer "F.Cu") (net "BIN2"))
 (segment (start 132.62 34.105585) (end 134.484415 35.97) (width 0.2) (layer "F.Cu") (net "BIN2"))
 (segment (start 134.484415 35.97) (end 140.379365 35.97) (width 0.2) (layer "F.Cu") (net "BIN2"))
 (segment (start 142.989365 38.58) (end 143.560635 38.58) (width 0.2) (layer "F.Cu") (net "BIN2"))
 (segment (start 116.931358 31.56) (end 131.565585 31.56) (width 0.2) (layer "F.Cu") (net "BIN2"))
 (segment (start 101.94 40.52) (end 107.971358 40.52) (width 0.2) (layer "F.Cu") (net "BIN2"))
 (segment (start 131.565585 31.56) (end 132.62 32.614415) (width 0.2) (layer "F.Cu") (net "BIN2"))
 (segment (start 107.971358 40.52) (end 116.931358 31.56) (width 0.2) (layer "F.Cu") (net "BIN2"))
 (via (at 144.76 41.03) (size 0.6) (drill 0.3) (layers "F.Cu" "B.Cu") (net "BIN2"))
 (segment (start 144.76 41.03) (end 144.76 41.335) (width 0.2) (layer "B.Cu") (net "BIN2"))
 (segment (start 144.76 41.335) (end 150.725 47.3) (width 0.2) (layer "B.Cu") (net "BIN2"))
 (segment (start 104.67 50.87) (end 120.99 50.87) (width 0.2) (layer "F.Cu") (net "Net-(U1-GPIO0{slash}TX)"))
 (segment (start 120.99 50.87) (end 129.62 42.24) (width 0.2) (layer "F.Cu") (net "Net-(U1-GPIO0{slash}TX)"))
 (segment (start 133.124315 36.46) (end 138.83 36.46) (width 0.2) (layer "F.Cu") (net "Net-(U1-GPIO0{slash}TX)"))
 (segment (start 129.62 42.24) (end 129.62 39.964315) (width 0.2) (layer "F.Cu") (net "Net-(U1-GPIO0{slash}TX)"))
 (segment (start 101.94 48.14) (end 104.67 50.87) (width 0.2) (layer "F.Cu") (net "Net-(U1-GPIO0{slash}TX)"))
 (segment (start 138.83 36.46) (end 139.73 37.36) (width 0.2) (layer "F.Cu") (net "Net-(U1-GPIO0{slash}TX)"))
 (segment (start 129.62 39.964315) (end 133.124315 36.46) (width 0.2) (layer "F.Cu") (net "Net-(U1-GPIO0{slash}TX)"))
 (segment (start 120.63 39.113654) (end 120.63 45.615) (width 0.2) (layer "F.Cu") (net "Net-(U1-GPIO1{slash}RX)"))
 (segment (start 131.51 37.15) (end 131.22 37.44) (width 0.2) (layer "F.Cu") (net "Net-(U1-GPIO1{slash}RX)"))
 (segment (start 122.656346 37.8) (end 121.943654 37.8) (width 0.2) (layer "F.Cu") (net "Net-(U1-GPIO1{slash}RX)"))
 (segment (start 120.63 45.615) (end 118.105 48.14) (width 0.2) (layer "F.Cu") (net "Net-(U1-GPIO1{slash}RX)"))
 (segment (start 123.016346 37.44) (end 122.656346 37.8) (width 0.2) (layer "F.Cu") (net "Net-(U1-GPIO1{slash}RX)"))
 (segment (start 121.943654 37.8) (end 120.63 39.113654) (width 0.2) (layer "F.Cu") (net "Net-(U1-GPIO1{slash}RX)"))
 (segment (start 131.22 37.44) (end 123.016346 37.44) (width 0.2) (layer "F.Cu") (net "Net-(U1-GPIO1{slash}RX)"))
 (via (at 131.51 37.15) (size 0.6) (drill 0.3) (layers "F.Cu" "B.Cu") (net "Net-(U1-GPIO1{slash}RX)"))
 (segment (start 131.51 37.75) (end 131.51 37.15) (width 0.2) (layer "B.Cu") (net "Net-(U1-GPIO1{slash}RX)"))
 (segment (start 133.66 39.9) (end 131.51 37.75) (width 0.2) (layer "B.Cu") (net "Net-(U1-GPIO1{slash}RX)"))
 (segment (start 139.73 39.9) (end 133.66 39.9) (width 0.2) (layer "B.Cu") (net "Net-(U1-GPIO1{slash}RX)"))
 (segment (start 131.666346 36.023654) (end 126.54 41.15) (width 0.2) (layer "B.Cu") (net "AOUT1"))
 (segment (start 141.681346 36.023654) (end 131.666346 36.023654) (width 0.2) (layer "B.Cu") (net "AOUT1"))
 (segment (start 143.105 34.6) (end 141.681346 36.023654) (width 0.2) (layer "B.Cu") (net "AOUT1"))
 (segment (start 136.925 45.86) (end 143.105 39.68) (width 0.2) (layer "B.Cu") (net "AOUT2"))
 (segment (start 128.71 45.86) (end 136.925 45.86) (width 0.2) (layer "B.Cu") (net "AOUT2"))
 (segment (start 126.54 43.69) (end 128.71 45.86) (width 0.2) (layer "B.Cu") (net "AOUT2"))
 (segment (start 143.220635 45.86) (end 142.649365 45.86) (width 0.2) (layer "F.Cu") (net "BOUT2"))
 (segment (start 142.005 43.32) (end 143.105 42.22) (width 0.2) (layer "F.Cu") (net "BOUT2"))
 (segment (start 144.270635 47.69) (end 144.270635 46.91) (width 0.2) (layer "F.Cu") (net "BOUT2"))
 (segment (start 144.270635 46.91) (end 143.220635 45.86) (width 0.2) (layer "F.Cu") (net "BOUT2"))
 (segment (start 135.54 48.4) (end 143.560635 48.4) (width 0.2) (layer "F.Cu") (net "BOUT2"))
 (segment (start 130.77 43.63) (end 135.54 48.4) (width 0.2) (layer "F.Cu") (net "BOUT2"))
 (segment (start 142.649365 45.86) (end 142.005 45.215635) (width 0.2) (layer "F.Cu") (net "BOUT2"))
 (segment (start 142.005 45.215635) (end 142.005 43.32) (width 0.2) (layer "F.Cu") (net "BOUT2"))
 (segment (start 143.560635 48.4) (end 144.270635 47.69) (width 0.2) (layer "F.Cu") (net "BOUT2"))
 (segment (start 136.28 36.86) (end 133.29 36.86) (width 0.2) (layer "F.Cu") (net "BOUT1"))
 (segment (start 133.29 36.86) (end 130.77 39.38) (width 0.2) (layer "F.Cu") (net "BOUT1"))
 (segment (start 130.77 39.38) (end 130.77 41.09) (width 0.2) (layer "F.Cu") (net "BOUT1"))
 (segment (start 137.2 41.395) (end 137.2 37.78) (width 0.2) (layer "F.Cu") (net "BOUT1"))
 (segment (start 137.2 37.78) (end 136.28 36.86) (width 0.2) (layer "F.Cu") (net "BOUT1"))
 (segment (start 143.105 47.3) (end 137.2 41.395) (width 0.2) (layer "F.Cu") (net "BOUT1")))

